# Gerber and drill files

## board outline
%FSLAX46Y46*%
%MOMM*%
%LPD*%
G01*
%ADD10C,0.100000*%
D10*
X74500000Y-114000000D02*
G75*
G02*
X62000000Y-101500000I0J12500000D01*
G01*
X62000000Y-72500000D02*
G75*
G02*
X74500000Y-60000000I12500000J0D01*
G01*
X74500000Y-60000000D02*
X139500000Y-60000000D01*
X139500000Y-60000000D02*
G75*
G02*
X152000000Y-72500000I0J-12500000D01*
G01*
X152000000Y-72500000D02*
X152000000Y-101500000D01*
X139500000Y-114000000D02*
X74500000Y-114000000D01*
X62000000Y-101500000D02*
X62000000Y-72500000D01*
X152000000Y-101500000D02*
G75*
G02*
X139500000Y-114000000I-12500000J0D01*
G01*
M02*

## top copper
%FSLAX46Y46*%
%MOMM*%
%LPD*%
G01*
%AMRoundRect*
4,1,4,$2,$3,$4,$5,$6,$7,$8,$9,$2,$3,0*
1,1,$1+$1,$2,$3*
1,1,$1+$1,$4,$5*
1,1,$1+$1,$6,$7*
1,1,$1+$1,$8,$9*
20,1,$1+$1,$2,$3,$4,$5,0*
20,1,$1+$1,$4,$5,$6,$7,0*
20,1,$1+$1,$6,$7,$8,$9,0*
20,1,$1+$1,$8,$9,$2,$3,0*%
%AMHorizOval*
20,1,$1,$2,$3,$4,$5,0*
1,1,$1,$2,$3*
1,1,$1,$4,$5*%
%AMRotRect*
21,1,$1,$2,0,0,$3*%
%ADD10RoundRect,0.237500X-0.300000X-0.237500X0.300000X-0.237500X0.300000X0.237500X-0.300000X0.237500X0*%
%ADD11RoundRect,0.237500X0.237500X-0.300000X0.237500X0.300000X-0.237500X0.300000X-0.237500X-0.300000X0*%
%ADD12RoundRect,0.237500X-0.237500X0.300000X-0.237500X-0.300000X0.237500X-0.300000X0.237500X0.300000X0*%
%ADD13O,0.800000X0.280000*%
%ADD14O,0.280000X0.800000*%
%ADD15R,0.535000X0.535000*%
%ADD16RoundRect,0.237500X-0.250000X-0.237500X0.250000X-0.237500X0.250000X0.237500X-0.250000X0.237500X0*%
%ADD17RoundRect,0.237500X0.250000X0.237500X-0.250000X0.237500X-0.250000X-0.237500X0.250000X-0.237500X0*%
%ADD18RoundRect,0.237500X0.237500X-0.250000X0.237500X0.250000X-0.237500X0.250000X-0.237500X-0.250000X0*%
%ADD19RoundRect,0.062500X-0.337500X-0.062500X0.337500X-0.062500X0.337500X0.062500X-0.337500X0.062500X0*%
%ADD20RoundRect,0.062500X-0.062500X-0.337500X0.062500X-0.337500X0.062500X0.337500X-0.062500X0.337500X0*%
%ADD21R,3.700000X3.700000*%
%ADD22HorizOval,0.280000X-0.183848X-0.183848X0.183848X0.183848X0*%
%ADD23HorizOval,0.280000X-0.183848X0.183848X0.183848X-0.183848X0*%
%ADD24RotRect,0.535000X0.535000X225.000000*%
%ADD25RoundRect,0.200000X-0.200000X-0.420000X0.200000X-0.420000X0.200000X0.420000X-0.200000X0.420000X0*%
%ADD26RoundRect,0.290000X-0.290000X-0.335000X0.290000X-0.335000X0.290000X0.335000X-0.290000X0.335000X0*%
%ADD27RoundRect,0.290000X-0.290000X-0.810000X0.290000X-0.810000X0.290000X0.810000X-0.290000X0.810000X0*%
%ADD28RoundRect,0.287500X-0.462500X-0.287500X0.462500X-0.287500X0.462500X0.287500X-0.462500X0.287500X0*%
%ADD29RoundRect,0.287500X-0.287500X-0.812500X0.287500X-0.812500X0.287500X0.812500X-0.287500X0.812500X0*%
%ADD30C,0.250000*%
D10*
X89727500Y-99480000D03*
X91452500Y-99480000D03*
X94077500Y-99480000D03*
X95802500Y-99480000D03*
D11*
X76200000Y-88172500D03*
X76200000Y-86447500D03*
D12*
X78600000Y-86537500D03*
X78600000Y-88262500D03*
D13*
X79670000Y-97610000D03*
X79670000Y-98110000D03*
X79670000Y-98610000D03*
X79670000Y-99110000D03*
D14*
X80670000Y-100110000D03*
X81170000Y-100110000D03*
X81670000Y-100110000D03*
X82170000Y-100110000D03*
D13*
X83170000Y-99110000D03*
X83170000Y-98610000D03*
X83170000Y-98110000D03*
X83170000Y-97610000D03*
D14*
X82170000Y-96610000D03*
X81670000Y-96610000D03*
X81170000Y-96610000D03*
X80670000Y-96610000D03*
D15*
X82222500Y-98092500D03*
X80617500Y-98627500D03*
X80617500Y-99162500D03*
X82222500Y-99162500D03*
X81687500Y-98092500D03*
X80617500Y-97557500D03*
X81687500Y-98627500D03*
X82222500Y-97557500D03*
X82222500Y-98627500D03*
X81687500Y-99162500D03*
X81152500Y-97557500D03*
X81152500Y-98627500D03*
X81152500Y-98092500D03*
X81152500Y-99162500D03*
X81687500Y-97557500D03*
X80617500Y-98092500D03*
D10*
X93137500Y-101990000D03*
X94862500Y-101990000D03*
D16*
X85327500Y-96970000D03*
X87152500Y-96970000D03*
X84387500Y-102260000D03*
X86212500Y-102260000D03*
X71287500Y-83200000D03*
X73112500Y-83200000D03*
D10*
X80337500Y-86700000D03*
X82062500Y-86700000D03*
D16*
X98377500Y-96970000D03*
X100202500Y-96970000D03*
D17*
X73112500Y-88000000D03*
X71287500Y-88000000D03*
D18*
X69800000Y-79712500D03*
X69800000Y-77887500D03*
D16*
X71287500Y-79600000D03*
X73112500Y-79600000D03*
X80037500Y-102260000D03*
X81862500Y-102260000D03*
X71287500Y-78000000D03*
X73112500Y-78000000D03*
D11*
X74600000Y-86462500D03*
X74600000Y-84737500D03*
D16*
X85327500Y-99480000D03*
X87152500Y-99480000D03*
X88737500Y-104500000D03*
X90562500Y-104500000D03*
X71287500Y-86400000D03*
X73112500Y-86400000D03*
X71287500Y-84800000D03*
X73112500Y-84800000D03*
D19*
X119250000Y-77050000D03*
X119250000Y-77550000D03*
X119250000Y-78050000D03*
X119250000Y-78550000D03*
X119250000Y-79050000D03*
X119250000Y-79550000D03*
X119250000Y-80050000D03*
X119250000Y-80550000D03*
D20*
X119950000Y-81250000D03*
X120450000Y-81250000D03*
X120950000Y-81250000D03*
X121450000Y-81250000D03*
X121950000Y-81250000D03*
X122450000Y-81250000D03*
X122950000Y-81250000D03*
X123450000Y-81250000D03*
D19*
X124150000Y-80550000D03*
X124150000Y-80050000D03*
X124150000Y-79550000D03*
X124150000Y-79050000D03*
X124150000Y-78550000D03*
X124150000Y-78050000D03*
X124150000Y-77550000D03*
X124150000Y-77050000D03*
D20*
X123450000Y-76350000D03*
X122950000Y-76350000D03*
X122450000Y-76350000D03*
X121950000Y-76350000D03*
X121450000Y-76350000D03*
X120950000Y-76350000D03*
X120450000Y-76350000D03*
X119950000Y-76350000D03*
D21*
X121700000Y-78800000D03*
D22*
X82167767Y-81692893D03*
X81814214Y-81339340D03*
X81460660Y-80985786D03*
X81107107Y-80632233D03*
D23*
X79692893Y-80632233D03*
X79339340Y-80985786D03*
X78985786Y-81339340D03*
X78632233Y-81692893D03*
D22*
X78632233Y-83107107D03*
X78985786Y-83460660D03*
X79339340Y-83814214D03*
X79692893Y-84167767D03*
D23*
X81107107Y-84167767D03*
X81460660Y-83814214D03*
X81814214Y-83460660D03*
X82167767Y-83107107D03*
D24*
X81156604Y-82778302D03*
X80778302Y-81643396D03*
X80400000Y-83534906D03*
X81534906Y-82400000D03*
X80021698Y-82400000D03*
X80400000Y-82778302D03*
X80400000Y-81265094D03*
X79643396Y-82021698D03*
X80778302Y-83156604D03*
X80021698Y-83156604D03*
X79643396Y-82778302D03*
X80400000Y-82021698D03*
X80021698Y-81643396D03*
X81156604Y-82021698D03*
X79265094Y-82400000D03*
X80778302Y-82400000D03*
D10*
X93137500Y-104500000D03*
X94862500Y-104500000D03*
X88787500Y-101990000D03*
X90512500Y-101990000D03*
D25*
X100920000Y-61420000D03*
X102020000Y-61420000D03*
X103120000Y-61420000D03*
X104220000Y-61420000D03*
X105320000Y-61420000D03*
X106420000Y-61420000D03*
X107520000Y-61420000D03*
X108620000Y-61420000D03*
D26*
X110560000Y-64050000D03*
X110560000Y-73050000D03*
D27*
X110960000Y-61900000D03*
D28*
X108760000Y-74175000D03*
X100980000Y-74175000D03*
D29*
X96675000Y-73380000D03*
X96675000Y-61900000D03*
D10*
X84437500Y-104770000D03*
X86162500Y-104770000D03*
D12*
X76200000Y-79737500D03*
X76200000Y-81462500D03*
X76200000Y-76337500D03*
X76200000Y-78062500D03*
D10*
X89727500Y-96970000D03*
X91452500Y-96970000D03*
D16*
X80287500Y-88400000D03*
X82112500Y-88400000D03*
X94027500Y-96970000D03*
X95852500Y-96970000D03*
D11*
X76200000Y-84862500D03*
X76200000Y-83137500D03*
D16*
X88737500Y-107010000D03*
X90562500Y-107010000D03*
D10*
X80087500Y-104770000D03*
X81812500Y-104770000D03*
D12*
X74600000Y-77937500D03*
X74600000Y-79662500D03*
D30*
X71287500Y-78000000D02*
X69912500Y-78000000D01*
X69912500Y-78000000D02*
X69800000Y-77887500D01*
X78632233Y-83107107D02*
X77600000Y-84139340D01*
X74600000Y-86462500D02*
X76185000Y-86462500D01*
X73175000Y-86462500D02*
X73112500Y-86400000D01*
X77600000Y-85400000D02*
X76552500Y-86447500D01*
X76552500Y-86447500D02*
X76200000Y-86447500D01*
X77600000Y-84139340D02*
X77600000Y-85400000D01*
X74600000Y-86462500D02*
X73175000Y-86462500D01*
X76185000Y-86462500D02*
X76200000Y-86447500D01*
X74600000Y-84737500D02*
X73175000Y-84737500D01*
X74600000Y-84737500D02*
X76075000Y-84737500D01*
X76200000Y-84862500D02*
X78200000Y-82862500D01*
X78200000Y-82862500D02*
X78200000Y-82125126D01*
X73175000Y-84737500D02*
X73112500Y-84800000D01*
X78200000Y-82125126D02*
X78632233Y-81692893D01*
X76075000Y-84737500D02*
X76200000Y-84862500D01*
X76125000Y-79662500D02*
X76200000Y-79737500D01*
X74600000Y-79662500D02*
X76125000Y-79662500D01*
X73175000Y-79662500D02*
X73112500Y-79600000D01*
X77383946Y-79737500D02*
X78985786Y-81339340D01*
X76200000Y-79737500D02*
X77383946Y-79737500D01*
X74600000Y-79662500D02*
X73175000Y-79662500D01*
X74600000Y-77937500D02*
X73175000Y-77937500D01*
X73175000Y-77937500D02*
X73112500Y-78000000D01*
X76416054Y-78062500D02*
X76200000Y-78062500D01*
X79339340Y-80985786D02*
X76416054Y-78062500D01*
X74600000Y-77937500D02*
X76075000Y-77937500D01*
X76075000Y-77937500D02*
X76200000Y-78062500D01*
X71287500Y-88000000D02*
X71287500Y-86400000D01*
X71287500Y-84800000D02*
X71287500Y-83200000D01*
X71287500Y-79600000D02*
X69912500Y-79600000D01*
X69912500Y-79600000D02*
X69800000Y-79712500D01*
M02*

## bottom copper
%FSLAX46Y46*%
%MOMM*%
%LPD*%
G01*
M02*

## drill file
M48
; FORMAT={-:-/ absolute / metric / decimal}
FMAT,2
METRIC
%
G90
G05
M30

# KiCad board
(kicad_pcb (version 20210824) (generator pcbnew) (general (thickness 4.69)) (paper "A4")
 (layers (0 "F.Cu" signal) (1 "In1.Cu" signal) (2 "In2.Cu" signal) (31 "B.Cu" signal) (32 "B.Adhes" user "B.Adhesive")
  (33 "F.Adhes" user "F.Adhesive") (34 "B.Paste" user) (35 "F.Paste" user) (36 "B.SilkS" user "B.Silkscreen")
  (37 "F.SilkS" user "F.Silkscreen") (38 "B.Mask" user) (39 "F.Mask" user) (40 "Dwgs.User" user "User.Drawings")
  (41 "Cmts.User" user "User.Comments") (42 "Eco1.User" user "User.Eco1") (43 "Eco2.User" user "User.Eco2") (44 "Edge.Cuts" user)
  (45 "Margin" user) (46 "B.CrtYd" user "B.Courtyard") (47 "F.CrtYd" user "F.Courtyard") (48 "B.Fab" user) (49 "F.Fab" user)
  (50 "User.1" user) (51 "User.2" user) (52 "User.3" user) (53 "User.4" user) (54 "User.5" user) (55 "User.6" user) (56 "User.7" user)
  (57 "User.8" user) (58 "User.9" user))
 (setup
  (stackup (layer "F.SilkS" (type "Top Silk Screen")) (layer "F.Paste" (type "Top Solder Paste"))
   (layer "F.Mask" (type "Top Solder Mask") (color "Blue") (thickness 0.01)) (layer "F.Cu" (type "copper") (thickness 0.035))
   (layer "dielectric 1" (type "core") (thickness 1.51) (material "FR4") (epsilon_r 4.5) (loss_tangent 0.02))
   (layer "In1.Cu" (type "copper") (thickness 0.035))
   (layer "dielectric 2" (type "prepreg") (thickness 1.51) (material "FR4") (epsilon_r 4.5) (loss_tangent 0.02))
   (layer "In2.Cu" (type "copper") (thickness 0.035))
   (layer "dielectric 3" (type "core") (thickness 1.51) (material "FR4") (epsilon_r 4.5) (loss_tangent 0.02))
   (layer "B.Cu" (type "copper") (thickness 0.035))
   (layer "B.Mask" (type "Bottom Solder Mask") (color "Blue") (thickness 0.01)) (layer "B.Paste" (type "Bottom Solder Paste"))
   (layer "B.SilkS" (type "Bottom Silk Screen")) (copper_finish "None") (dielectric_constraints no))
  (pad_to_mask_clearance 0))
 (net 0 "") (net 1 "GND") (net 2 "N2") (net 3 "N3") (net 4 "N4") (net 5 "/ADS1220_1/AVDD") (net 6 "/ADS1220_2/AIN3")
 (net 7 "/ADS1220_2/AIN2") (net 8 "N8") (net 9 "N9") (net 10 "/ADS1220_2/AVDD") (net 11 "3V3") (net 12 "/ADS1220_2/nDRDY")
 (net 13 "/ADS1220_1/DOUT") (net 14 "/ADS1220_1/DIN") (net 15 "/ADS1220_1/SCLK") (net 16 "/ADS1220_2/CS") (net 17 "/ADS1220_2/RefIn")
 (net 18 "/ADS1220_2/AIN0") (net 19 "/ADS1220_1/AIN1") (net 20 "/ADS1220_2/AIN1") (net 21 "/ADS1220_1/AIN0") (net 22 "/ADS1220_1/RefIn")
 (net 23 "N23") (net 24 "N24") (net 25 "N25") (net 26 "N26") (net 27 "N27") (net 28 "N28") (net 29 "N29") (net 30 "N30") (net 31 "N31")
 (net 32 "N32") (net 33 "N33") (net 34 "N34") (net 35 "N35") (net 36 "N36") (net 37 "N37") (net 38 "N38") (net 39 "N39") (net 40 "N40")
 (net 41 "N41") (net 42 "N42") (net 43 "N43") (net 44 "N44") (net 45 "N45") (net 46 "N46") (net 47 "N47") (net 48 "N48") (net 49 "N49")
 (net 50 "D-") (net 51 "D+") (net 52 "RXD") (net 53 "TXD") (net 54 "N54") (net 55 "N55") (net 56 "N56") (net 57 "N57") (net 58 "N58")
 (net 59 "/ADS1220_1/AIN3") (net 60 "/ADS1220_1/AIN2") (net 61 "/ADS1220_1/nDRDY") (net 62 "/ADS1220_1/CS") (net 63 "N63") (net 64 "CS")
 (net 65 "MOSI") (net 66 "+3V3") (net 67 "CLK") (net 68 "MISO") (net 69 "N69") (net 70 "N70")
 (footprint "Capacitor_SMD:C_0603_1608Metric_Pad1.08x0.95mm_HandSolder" (layer "F.Cu") (at 90.59 99.48)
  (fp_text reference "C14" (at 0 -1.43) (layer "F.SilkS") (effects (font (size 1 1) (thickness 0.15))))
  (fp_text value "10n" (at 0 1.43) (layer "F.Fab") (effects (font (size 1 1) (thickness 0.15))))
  (pad "1" smd roundrect locked (at -0.8625 0) (size 1.075 0.95) (layers "F.Cu" "F.Paste" "F.Mask") (roundrect_rratio 0.25) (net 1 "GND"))
  (pad "2" smd roundrect locked (at 0.8625 0) (size 1.075 0.95) (layers "F.Cu" "F.Paste" "F.Mask") (roundrect_rratio 0.25) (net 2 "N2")))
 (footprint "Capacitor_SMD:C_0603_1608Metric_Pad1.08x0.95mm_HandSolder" (layer "F.Cu") (at 94.94 99.48)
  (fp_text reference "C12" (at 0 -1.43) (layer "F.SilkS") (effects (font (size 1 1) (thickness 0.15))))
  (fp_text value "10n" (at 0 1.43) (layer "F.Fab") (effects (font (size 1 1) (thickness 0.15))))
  (pad "1" smd roundrect locked (at -0.8625 0) (size 1.075 0.95) (layers "F.Cu" "F.Paste" "F.Mask") (roundrect_rratio 0.25) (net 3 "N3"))
  (pad "2" smd roundrect locked (at 0.8625 0) (size 1.075 0.95) (layers "F.Cu" "F.Paste" "F.Mask") (roundrect_rratio 0.25) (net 1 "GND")))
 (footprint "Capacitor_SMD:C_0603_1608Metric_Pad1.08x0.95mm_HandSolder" (layer "F.Cu") (at 76.2 87.31 90)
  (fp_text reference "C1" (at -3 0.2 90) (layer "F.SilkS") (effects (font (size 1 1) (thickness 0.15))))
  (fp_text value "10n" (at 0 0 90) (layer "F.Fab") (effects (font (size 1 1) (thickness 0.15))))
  (pad "1" smd roundrect locked (at -0.8625 0 90) (size 1.075 0.95) (layers "F.Cu" "F.Paste" "F.Mask") (roundrect_rratio 0.25) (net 1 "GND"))
  (pad "2" smd roundrect locked (at 0.8625 0 90) (size 1.075 0.95) (layers "F.Cu" "F.Paste" "F.Mask") (roundrect_rratio 0.25) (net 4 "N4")))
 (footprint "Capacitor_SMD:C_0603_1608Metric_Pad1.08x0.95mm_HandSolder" (layer "F.Cu") (at 78.6 87.4 -90)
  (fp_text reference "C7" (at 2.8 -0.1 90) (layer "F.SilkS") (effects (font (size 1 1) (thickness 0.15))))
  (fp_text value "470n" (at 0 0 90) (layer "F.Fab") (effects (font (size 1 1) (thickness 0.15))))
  (pad "1" smd roundrect locked (at -0.8625 0 270) (size 1.075 0.95) (layers "F.Cu" "F.Paste" "F.Mask") (roundrect_rratio 0.25)
   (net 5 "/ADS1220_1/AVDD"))
  (pad "2" smd roundrect locked (at 0.8625 0 270) (size 1.075 0.95) (layers "F.Cu" "F.Paste" "F.Mask") (roundrect_rratio 0.25) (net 1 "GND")))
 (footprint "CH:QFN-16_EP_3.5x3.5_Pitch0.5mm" (layer "F.Cu") (at 81.42 98.36)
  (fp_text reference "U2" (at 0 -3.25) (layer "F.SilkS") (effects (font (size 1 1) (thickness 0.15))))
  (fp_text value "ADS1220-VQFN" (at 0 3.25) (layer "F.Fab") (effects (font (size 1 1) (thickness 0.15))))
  (pad "1" smd oval (at -1.75 -0.75 90) (size 0.28 0.8) (layers "F.Cu" "F.Paste" "F.Mask") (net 1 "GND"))
  (pad "2" smd oval (at -1.75 -0.25 90) (size 0.28 0.8) (layers "F.Cu" "F.Paste" "F.Mask") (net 1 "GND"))
  (pad "3" smd oval (at -1.75 0.25 90) (size 0.28 0.8) (layers "F.Cu" "F.Paste" "F.Mask") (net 1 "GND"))
  (pad "4" smd oval (at -1.75 0.75 90) (size 0.28 0.8) (layers "F.Cu" "F.Paste" "F.Mask") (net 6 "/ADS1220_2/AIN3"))
  (pad "5" smd oval (at -0.75 1.75) (size 0.28 0.8) (layers "F.Cu" "F.Paste" "F.Mask") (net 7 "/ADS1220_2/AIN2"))
  (pad "6" smd oval (at -0.25 1.75) (size 0.28 0.8) (layers "F.Cu" "F.Paste" "F.Mask") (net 2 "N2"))
  (pad "7" smd oval (at 0.25 1.75) (size 0.28 0.8) (layers "F.Cu" "F.Paste" "F.Mask") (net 3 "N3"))
  (pad "8" smd oval (at 0.75 1.75) (size 0.28 0.8) (layers "F.Cu" "F.Paste" "F.Mask") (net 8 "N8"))
  (pad "9" smd oval (at 1.75 0.75 90) (size 0.28 0.8) (layers "F.Cu" "F.Paste" "F.Mask") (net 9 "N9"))
  (pad "10" smd oval (at 1.75 0.25 90) (size 0.28 0.8) (layers "F.Cu" "F.Paste" "F.Mask") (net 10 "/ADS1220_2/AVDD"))
  (pad "11" smd oval (at 1.75 -0.25 90) (size 0.28 0.8) (layers "F.Cu" "F.Paste" "F.Mask") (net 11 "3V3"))
  (pad "12" smd oval (at 1.75 -0.75 90) (size 0.28 0.8) (layers "F.Cu" "F.Paste" "F.Mask") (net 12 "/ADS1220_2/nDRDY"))
  (pad "13" smd oval (at 0.75 -1.75) (size 0.28 0.8) (layers "F.Cu" "F.Paste" "F.Mask") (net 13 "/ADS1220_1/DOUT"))
  (pad "14" smd oval (at 0.25 -1.75) (size 0.28 0.8) (layers "F.Cu" "F.Paste" "F.Mask") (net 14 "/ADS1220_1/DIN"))
  (pad "15" smd oval (at -0.25 -1.75) (size 0.28 0.8) (layers "F.Cu" "F.Paste" "F.Mask") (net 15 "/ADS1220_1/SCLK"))
  (pad "16" smd oval (at -0.75 -1.75) (size 0.28 0.8) (layers "F.Cu" "F.Paste" "F.Mask") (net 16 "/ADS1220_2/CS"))
  (pad "17" smd rect (at 0.8025 -0.2675) (size 0.535 0.535) (layers "F.Cu" "F.Paste" "F.Mask") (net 1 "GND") (solder_paste_margin -0.75))
  (pad "17" smd rect (at -0.8025 0.2675) (size 0.535 0.535) (layers "F.Cu" "F.Paste" "F.Mask") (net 1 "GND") (solder_paste_margin -0.75))
  (pad "17" smd rect (at -0.8025 0.8025) (size 0.535 0.535) (layers "F.Cu" "F.Paste" "F.Mask") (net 1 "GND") (solder_paste_margin -0.75))
  (pad "17" smd rect (at 0.8025 0.8025) (size 0.535 0.535) (layers "F.Cu" "F.Paste" "F.Mask") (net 1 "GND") (solder_paste_margin -0.75))
  (pad "17" smd rect (at 0.2675 -0.2675) (size 0.535 0.535) (layers "F.Cu" "F.Paste" "F.Mask") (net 1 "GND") (solder_paste_margin -0.75))
  (pad "17" smd rect (at -0.8025 -0.8025) (size 0.535 0.535) (layers "F.Cu" "F.Paste" "F.Mask") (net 1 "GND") (solder_paste_margin -0.75))
  (pad "17" smd rect (at 0.2675 0.2675) (size 0.535 0.535) (layers "F.Cu" "F.Paste" "F.Mask") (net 1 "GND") (solder_paste_margin -0.75))
  (pad "17" smd rect (at 0.8025 -0.8025) (size 0.535 0.535) (layers "F.Cu" "F.Paste" "F.Mask") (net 1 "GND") (solder_paste_margin -0.75))
  (pad "17" smd rect (at 0.8025 0.2675) (size 0.535 0.535) (layers "F.Cu" "F.Paste" "F.Mask") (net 1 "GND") (solder_paste_margin -0.75))
  (pad "17" smd rect (at 0.2675 0.8025) (size 0.535 0.535) (layers "F.Cu" "F.Paste" "F.Mask") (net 1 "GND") (solder_paste_margin -0.75))
  (pad "17" smd rect (at -0.2675 -0.8025) (size 0.535 0.535) (layers "F.Cu" "F.Paste" "F.Mask") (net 1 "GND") (solder_paste_margin -0.75))
  (pad "17" smd rect (at -0.2675 0.2675) (size 0.535 0.535) (layers "F.Cu" "F.Paste" "F.Mask") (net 1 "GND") (solder_paste_margin -0.75))
  (pad "17" smd rect (at -0.2675 -0.2675) (size 0.535 0.535) (layers "F.Cu" "F.Paste" "F.Mask") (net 1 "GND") (solder_paste_margin -0.75))
  (pad "17" smd rect (at -0.2675 0.8025) (size 0.535 0.535) (layers "F.Cu" "F.Paste" "F.Mask") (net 1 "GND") (solder_paste_margin -0.75))
  (pad "17" smd rect (at 0.2675 -0.8025) (size 0.535 0.535) (layers "F.Cu" "F.Paste" "F.Mask") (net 1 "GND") (solder_paste_margin -0.75))
  (pad "17" smd rect (at -0.8025 -0.2675) (size 0.535 0.535) (layers "F.Cu" "F.Paste" "F.Mask") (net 1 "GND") (solder_paste_margin -0.75)))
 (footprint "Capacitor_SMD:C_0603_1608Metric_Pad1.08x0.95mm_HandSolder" (layer "F.Cu") (at 94 101.99)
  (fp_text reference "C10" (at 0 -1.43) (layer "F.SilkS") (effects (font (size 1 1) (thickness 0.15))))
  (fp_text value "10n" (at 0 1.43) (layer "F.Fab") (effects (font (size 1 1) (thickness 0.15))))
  (pad "1" smd roundrect locked (at -0.8625 0) (size 1.075 0.95) (layers "F.Cu" "F.Paste" "F.Mask") (roundrect_rratio 0.25) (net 8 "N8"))
  (pad "2" smd roundrect locked (at 0.8625 0) (size 1.075 0.95) (layers "F.Cu" "F.Paste" "F.Mask") (roundrect_rratio 0.25) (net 1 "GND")))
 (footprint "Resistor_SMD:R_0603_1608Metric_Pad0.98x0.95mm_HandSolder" (layer "F.Cu") (at 86.24 96.97)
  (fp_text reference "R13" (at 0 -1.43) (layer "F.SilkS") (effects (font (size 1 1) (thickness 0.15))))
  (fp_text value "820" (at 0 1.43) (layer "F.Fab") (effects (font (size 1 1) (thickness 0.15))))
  (pad "1" smd roundrect locked (at -0.9125 0) (size 0.975 0.95) (layers "F.Cu" "F.Paste" "F.Mask") (roundrect_rratio 0.25)
   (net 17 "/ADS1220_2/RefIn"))
  (pad "2" smd roundrect locked (at 0.9125 0) (size 0.975 0.95) (layers "F.Cu" "F.Paste" "F.Mask") (roundrect_rratio 0.25) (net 3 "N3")))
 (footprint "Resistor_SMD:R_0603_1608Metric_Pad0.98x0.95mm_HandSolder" (layer "F.Cu") (at 85.3 102.26)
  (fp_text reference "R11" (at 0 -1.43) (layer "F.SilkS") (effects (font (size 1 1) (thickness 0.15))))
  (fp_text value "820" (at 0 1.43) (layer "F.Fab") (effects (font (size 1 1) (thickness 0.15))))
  (pad "1" smd roundrect locked (at -0.9125 0) (size 0.975 0.95) (layers "F.Cu" "F.Paste" "F.Mask") (roundrect_rratio 0.25)
   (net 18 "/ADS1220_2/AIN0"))
  (pad "2" smd roundrect locked (at 0.9125 0) (size 0.975 0.95) (layers "F.Cu" "F.Paste" "F.Mask") (roundrect_rratio 0.25) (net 9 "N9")))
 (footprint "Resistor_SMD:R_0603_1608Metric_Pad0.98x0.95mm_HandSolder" (layer "F.Cu") (at 72.2 83.2)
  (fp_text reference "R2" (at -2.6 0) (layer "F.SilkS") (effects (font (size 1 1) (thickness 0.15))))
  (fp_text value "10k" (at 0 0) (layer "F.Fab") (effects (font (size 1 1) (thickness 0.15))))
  (pad "1" smd roundrect locked (at -0.9125 0) (size 0.975 0.95) (layers "F.Cu" "F.Paste" "F.Mask") (roundrect_rratio 0.25)
   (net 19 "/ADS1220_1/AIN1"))
  (pad "2" smd roundrect locked (at 0.9125 0) (size 0.975 0.95) (layers "F.Cu" "F.Paste" "F.Mask") (roundrect_rratio 0.25) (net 1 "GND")))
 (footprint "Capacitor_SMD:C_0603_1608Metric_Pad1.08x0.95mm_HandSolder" (layer "F.Cu") (at 81.2 86.7)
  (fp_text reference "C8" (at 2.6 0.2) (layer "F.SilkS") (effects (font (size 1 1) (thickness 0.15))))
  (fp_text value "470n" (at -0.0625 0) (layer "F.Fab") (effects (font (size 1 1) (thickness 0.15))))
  (pad "1" smd roundrect locked (at -0.8625 0) (size 1.075 0.95) (layers "F.Cu" "F.Paste" "F.Mask") (roundrect_rratio 0.25) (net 11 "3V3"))
  (pad "2" smd roundrect locked (at 0.8625 0) (size 1.075 0.95) (layers "F.Cu" "F.Paste" "F.Mask") (roundrect_rratio 0.25) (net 1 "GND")))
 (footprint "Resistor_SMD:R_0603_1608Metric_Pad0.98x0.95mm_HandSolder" (layer "F.Cu") (at 99.29 96.97)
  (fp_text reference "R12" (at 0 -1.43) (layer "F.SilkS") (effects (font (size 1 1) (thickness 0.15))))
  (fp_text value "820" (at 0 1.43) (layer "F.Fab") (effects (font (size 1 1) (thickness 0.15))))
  (pad "1" smd roundrect locked (at -0.9125 0) (size 0.975 0.95) (layers "F.Cu" "F.Paste" "F.Mask") (roundrect_rratio 0.25)
   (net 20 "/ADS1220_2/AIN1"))
  (pad "2" smd roundrect locked (at 0.9125 0) (size 0.975 0.95) (layers "F.Cu" "F.Paste" "F.Mask") (roundrect_rratio 0.25) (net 8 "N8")))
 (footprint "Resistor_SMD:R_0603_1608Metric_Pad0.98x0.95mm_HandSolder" (layer "F.Cu") (at 72.2 88 180)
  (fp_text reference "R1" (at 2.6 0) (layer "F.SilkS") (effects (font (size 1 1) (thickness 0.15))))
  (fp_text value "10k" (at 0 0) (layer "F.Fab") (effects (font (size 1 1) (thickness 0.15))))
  (pad "1" smd roundrect locked (at -0.9125 0 180) (size 0.975 0.95) (layers "F.Cu" "F.Paste" "F.Mask") (roundrect_rratio 0.25)
   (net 5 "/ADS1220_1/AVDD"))
  (pad "2" smd roundrect locked (at 0.9125 0 180) (size 0.975 0.95) (layers "F.Cu" "F.Paste" "F.Mask") (roundrect_rratio 0.25)
   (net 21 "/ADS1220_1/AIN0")))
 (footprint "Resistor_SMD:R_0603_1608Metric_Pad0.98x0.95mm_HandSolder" (layer "F.Cu") (at 69.8 78.8 90)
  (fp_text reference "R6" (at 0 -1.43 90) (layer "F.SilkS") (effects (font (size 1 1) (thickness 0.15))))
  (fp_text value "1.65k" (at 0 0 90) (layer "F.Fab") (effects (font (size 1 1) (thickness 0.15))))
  (pad "1" smd roundrect locked (at -0.9125 0 90) (size 0.975 0.95) (layers "F.Cu" "F.Paste" "F.Mask") (roundrect_rratio 0.25)
   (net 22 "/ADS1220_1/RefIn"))
  (pad "2" smd roundrect locked (at 0.9125 0 90) (size 0.975 0.95) (layers "F.Cu" "F.Paste" "F.Mask") (roundrect_rratio 0.25) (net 1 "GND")))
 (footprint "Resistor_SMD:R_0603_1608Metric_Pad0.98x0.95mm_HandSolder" (layer "F.Cu") (at 72.2 79.6)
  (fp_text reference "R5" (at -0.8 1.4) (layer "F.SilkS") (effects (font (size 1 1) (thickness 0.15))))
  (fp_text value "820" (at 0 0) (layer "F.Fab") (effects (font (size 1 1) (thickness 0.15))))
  (pad "1" smd roundrect locked (at -0.9125 0) (size 0.975 0.95) (layers "F.Cu" "F.Paste" "F.Mask") (roundrect_rratio 0.25)
   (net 22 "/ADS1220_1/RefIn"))
  (pad "2" smd roundrect locked (at 0.9125 0) (size 0.975 0.95) (layers "F.Cu" "F.Paste" "F.Mask") (roundrect_rratio 0.25) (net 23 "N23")))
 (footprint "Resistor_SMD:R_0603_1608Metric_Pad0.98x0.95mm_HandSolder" (layer "F.Cu") (at 80.95 102.26)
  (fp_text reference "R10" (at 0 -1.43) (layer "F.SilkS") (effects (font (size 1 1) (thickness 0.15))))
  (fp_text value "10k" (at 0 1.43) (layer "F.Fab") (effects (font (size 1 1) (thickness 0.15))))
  (pad "1" smd roundrect locked (at -0.9125 0) (size 0.975 0.95) (layers "F.Cu" "F.Paste" "F.Mask") (roundrect_rratio 0.25)
   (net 20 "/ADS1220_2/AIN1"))
  (pad "2" smd roundrect locked (at 0.9125 0) (size 0.975 0.95) (layers "F.Cu" "F.Paste" "F.Mask") (roundrect_rratio 0.25) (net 1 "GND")))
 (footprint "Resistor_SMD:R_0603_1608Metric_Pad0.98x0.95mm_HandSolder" (layer "F.Cu") (at 72.2 78)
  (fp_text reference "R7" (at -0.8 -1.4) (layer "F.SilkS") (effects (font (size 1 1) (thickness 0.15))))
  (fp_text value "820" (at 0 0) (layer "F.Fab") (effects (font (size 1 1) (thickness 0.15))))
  (pad "1" smd roundrect locked (at -0.9125 0) (size 0.975 0.95) (layers "F.Cu" "F.Paste" "F.Mask") (roundrect_rratio 0.25) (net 1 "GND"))
  (pad "2" smd roundrect locked (at 0.9125 0) (size 0.975 0.95) (layers "F.Cu" "F.Paste" "F.Mask") (roundrect_rratio 0.25) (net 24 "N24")))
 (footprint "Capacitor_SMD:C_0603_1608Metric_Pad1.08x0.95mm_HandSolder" (layer "F.Cu") (at 74.6 85.6 90)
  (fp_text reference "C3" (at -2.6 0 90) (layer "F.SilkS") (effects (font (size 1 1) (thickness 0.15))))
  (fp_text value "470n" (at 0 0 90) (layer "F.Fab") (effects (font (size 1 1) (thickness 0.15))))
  (pad "1" smd roundrect locked (at -0.8625 0 90) (size 1.075 0.95) (layers "F.Cu" "F.Paste" "F.Mask") (roundrect_rratio 0.25) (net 4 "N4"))
  (pad "2" smd roundrect locked (at 0.8625 0 90) (size 1.075 0.95) (layers "F.Cu" "F.Paste" "F.Mask") (roundrect_rratio 0.25) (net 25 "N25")))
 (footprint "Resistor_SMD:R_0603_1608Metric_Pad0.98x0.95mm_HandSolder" (layer "F.Cu") (at 86.24 99.48)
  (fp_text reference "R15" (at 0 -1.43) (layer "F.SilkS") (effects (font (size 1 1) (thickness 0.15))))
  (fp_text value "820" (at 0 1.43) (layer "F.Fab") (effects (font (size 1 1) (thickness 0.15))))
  (pad "1" smd roundrect locked (at -0.9125 0) (size 0.975 0.95) (layers "F.Cu" "F.Paste" "F.Mask") (roundrect_rratio 0.25) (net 1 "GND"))
  (pad "2" smd roundrect locked (at 0.9125 0) (size 0.975 0.95) (layers "F.Cu" "F.Paste" "F.Mask") (roundrect_rratio 0.25) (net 2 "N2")))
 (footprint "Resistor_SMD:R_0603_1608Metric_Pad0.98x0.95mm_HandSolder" (layer "F.Cu") (at 89.65 104.5)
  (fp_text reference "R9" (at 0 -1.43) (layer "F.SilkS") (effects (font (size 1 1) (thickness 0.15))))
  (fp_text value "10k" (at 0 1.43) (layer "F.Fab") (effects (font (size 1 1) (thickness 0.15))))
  (pad "1" smd roundrect locked (at -0.9125 0) (size 0.975 0.95) (layers "F.Cu" "F.Paste" "F.Mask") (roundrect_rratio 0.25)
   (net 10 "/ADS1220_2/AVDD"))
  (pad "2" smd roundrect locked (at 0.9125 0) (size 0.975 0.95) (layers "F.Cu" "F.Paste" "F.Mask") (roundrect_rratio 0.25)
   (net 18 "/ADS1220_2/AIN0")))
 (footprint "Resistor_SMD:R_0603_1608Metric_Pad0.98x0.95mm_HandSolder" (layer "F.Cu") (at 72.2 86.4)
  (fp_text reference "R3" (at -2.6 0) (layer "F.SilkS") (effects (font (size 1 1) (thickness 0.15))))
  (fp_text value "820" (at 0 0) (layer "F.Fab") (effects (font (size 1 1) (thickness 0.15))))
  (pad "1" smd roundrect locked (at -0.9125 0) (size 0.975 0.95) (layers "F.Cu" "F.Paste" "F.Mask") (roundrect_rratio 0.25)
   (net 21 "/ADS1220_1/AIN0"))
  (pad "2" smd roundrect locked (at 0.9125 0) (size 0.975 0.95) (layers "F.Cu" "F.Paste" "F.Mask") (roundrect_rratio 0.25) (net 4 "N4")))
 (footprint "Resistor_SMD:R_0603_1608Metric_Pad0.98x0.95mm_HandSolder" (layer "F.Cu") (at 72.2 84.8)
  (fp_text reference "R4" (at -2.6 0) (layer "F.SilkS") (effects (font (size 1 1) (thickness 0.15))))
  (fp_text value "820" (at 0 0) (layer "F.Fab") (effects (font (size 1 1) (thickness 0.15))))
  (pad "1" smd roundrect locked (at -0.9125 0) (size 0.975 0.95) (layers "F.Cu" "F.Paste" "F.Mask") (roundrect_rratio 0.25)
   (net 19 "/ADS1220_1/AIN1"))
  (pad "2" smd roundrect locked (at 0.9125 0) (size 0.975 0.95) (layers "F.Cu" "F.Paste" "F.Mask") (roundrect_rratio 0.25) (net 25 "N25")))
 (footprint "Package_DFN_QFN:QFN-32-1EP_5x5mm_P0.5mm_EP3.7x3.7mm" (layer "F.Cu") (at 121.7 78.8)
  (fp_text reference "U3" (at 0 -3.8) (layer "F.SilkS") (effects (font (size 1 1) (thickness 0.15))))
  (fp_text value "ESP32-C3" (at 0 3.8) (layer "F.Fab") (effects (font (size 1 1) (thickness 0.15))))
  (pad "" smd roundrect locked (at 0.925 -0.925) (size 1.49 1.49) (layers "F.Paste") (roundrect_rratio 0.167785))
  (pad "" smd roundrect locked (at -0.925 0.925) (size 1.49 1.49) (layers "F.Paste") (roundrect_rratio 0.167785))
  (pad "" smd roundrect locked (at -0.925 -0.925) (size 1.49 1.49) (layers "F.Paste") (roundrect_rratio 0.167785))
  (pad "" smd roundrect locked (at 0.925 0.925) (size 1.49 1.49) (layers "F.Paste") (roundrect_rratio 0.167785))
  (pad "1" smd roundrect locked (at -2.45 -1.75) (size 0.8 0.25) (layers "F.Cu" "F.Paste" "F.Mask") (roundrect_rratio 0.25) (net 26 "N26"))
  (pad "2" smd roundrect locked (at -2.45 -1.25) (size 0.8 0.25) (layers "F.Cu" "F.Paste" "F.Mask") (roundrect_rratio 0.25) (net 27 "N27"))
  (pad "3" smd roundrect locked (at -2.45 -0.75) (size 0.8 0.25) (layers "F.Cu" "F.Paste" "F.Mask") (roundrect_rratio 0.25) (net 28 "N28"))
  (pad "4" smd roundrect locked (at -2.45 -0.25) (size 0.8 0.25) (layers "F.Cu" "F.Paste" "F.Mask") (roundrect_rratio 0.25) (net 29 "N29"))
  (pad "5" smd roundrect locked (at -2.45 0.25) (size 0.8 0.25) (layers "F.Cu" "F.Paste" "F.Mask") (roundrect_rratio 0.25) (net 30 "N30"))
  (pad "6" smd roundrect locked (at -2.45 0.75) (size 0.8 0.25) (layers "F.Cu" "F.Paste" "F.Mask") (roundrect_rratio 0.25) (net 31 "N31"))
  (pad "7" smd roundrect locked (at -2.45 1.25) (size 0.8 0.25) (layers "F.Cu" "F.Paste" "F.Mask") (roundrect_rratio 0.25) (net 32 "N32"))
  (pad "8" smd roundrect locked (at -2.45 1.75) (size 0.8 0.25) (layers "F.Cu" "F.Paste" "F.Mask") (roundrect_rratio 0.25) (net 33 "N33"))
  (pad "9" smd roundrect locked (at -1.75 2.45) (size 0.25 0.8) (layers "F.Cu" "F.Paste" "F.Mask") (roundrect_rratio 0.25) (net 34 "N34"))
  (pad "10" smd roundrect locked (at -1.25 2.45) (size 0.25 0.8) (layers "F.Cu" "F.Paste" "F.Mask") (roundrect_rratio 0.25) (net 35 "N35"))
  (pad "11" smd roundrect locked (at -0.75 2.45) (size 0.25 0.8) (layers "F.Cu" "F.Paste" "F.Mask") (roundrect_rratio 0.25) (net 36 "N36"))
  (pad "12" smd roundrect locked (at -0.25 2.45) (size 0.25 0.8) (layers "F.Cu" "F.Paste" "F.Mask") (roundrect_rratio 0.25) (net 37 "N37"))
  (pad "13" smd roundrect locked (at 0.25 2.45) (size 0.25 0.8) (layers "F.Cu" "F.Paste" "F.Mask") (roundrect_rratio 0.25) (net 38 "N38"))
  (pad "14" smd roundrect locked (at 0.75 2.45) (size 0.25 0.8) (layers "F.Cu" "F.Paste" "F.Mask") (roundrect_rratio 0.25) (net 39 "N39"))
  (pad "15" smd roundrect locked (at 1.25 2.45) (size 0.25 0.8) (layers "F.Cu" "F.Paste" "F.Mask") (roundrect_rratio 0.25) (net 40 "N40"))
  (pad "16" smd roundrect locked (at 1.75 2.45) (size 0.25 0.8) (layers "F.Cu" "F.Paste" "F.Mask") (roundrect_rratio 0.25) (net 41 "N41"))
  (pad "17" smd roundrect locked (at 2.45 1.75) (size 0.8 0.25) (layers "F.Cu" "F.Paste" "F.Mask") (roundrect_rratio 0.25) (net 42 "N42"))
  (pad "18" smd roundrect locked (at 2.45 1.25) (size 0.8 0.25) (layers "F.Cu" "F.Paste" "F.Mask") (roundrect_rratio 0.25) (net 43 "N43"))
  (pad "19" smd roundrect locked (at 2.45 0.75) (size 0.8 0.25) (layers "F.Cu" "F.Paste" "F.Mask") (roundrect_rratio 0.25) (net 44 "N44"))
  (pad "20" smd roundrect locked (at 2.45 0.25) (size 0.8 0.25) (layers "F.Cu" "F.Paste" "F.Mask") (roundrect_rratio 0.25) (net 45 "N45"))
  (pad "21" smd roundrect locked (at 2.45 -0.25) (size 0.8 0.25) (layers "F.Cu" "F.Paste" "F.Mask") (roundrect_rratio 0.25) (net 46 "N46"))
  (pad "22" smd roundrect locked (at 2.45 -0.75) (size 0.8 0.25) (layers "F.Cu" "F.Paste" "F.Mask") (roundrect_rratio 0.25) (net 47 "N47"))
  (pad "23" smd roundrect locked (at 2.45 -1.25) (size 0.8 0.25) (layers "F.Cu" "F.Paste" "F.Mask") (roundrect_rratio 0.25) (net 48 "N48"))
  (pad "24" smd roundrect locked (at 2.45 -1.75) (size 0.8 0.25) (layers "F.Cu" "F.Paste" "F.Mask") (roundrect_rratio 0.25) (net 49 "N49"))
  (pad "25" smd roundrect locked (at 1.75 -2.45) (size 0.25 0.8) (layers "F.Cu" "F.Paste" "F.Mask") (roundrect_rratio 0.25) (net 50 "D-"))
  (pad "26" smd roundrect locked (at 1.25 -2.45) (size 0.25 0.8) (layers "F.Cu" "F.Paste" "F.Mask") (roundrect_rratio 0.25) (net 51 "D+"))
  (pad "27" smd roundrect locked (at 0.75 -2.45) (size 0.25 0.8) (layers "F.Cu" "F.Paste" "F.Mask") (roundrect_rratio 0.25) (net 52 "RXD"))
  (pad "28" smd roundrect locked (at 0.25 -2.45) (size 0.25 0.8) (layers "F.Cu" "F.Paste" "F.Mask") (roundrect_rratio 0.25) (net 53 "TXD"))
  (pad "29" smd roundrect locked (at -0.25 -2.45) (size 0.25 0.8) (layers "F.Cu" "F.Paste" "F.Mask") (roundrect_rratio 0.25) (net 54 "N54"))
  (pad "30" smd roundrect locked (at -0.75 -2.45) (size 0.25 0.8) (layers "F.Cu" "F.Paste" "F.Mask") (roundrect_rratio 0.25) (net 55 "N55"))
  (pad "31" smd roundrect locked (at -1.25 -2.45) (size 0.25 0.8) (layers "F.Cu" "F.Paste" "F.Mask") (roundrect_rratio 0.25) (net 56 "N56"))
  (pad "32" smd roundrect locked (at -1.75 -2.45) (size 0.25 0.8) (layers "F.Cu" "F.Paste" "F.Mask") (roundrect_rratio 0.25) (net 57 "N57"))
  (pad "33" smd rect locked (at 0 0) (size 3.7 3.7) (layers "F.Cu" "F.Mask") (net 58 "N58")))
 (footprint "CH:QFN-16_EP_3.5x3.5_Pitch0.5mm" (layer "F.Cu") (at 80.4 82.4 -135)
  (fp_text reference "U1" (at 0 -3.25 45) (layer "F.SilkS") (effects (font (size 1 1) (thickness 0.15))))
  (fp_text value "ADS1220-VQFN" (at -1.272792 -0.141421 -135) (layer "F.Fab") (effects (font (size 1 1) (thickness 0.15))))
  (pad "1" smd oval (at -1.75 -0.75 315) (size 0.28 0.8) (layers "F.Cu" "F.Paste" "F.Mask") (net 1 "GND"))
  (pad "2" smd oval (at -1.75 -0.25 315) (size 0.28 0.8) (layers "F.Cu" "F.Paste" "F.Mask") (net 1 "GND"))
  (pad "3" smd oval (at -1.75 0.25 315) (size 0.28 0.8) (layers "F.Cu" "F.Paste" "F.Mask") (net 1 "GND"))
  (pad "4" smd oval (at -1.75 0.75 315) (size 0.28 0.8) (layers "F.Cu" "F.Paste" "F.Mask") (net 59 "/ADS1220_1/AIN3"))
  (pad "5" smd oval (at -0.75 1.75 225) (size 0.28 0.8) (layers "F.Cu" "F.Paste" "F.Mask") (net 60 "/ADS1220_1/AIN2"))
  (pad "6" smd oval (at -0.25 1.75 225) (size 0.28 0.8) (layers "F.Cu" "F.Paste" "F.Mask") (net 24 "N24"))
  (pad "7" smd oval (at 0.25 1.75 225) (size 0.28 0.8) (layers "F.Cu" "F.Paste" "F.Mask") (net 23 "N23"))
  (pad "8" smd oval (at 0.75 1.75 225) (size 0.28 0.8) (layers "F.Cu" "F.Paste" "F.Mask") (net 25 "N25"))
  (pad "9" smd oval (at 1.75 0.75 315) (size 0.28 0.8) (layers "F.Cu" "F.Paste" "F.Mask") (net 4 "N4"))
  (pad "10" smd oval (at 1.75 0.25 315) (size 0.28 0.8) (layers "F.Cu" "F.Paste" "F.Mask") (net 5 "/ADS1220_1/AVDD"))
  (pad "11" smd oval (at 1.75 -0.25 315) (size 0.28 0.8) (layers "F.Cu" "F.Paste" "F.Mask") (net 11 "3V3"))
  (pad "12" smd oval (at 1.75 -0.75 315) (size 0.28 0.8) (layers "F.Cu" "F.Paste" "F.Mask") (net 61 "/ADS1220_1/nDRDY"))
  (pad "13" smd oval (at 0.75 -1.75 225) (size 0.28 0.8) (layers "F.Cu" "F.Paste" "F.Mask") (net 13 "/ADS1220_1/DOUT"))
  (pad "14" smd oval (at 0.25 -1.75 225) (size 0.28 0.8) (layers "F.Cu" "F.Paste" "F.Mask") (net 14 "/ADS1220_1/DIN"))
  (pad "15" smd oval (at -0.25 -1.75 225) (size 0.28 0.8) (layers "F.Cu" "F.Paste" "F.Mask") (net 15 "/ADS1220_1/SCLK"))
  (pad "16" smd oval (at -0.75 -1.75 225) (size 0.28 0.8) (layers "F.Cu" "F.Paste" "F.Mask") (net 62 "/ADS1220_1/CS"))
  (pad "17" smd rect (at -0.2675 -0.8025 225) (size 0.535 0.535) (layers "F.Cu" "F.Paste" "F.Mask") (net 1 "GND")
   (solder_paste_margin -0.75))
  (pad "17" smd rect (at -0.8025 0.2675 225) (size 0.535 0.535) (layers "F.Cu" "F.Paste" "F.Mask") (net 1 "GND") (solder_paste_margin -0.75))
  (pad "17" smd rect (at 0.8025 -0.8025 225) (size 0.535 0.535) (layers "F.Cu" "F.Paste" "F.Mask") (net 1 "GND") (solder_paste_margin -0.75))
  (pad "17" smd rect (at -0.8025 -0.8025 225) (size 0.535 0.535) (layers "F.Cu" "F.Paste" "F.Mask") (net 1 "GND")
   (solder_paste_margin -0.75))
  (pad "17" smd rect (at 0.2675 0.2675 225) (size 0.535 0.535) (layers "F.Cu" "F.Paste" "F.Mask") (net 1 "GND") (solder_paste_margin -0.75))
  (pad "17" smd rect (at 0.2675 -0.2675 225) (size 0.535 0.535) (layers "F.Cu" "F.Paste" "F.Mask") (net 1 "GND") (solder_paste_margin -0.75))
  (pad "17" smd rect (at -0.8025 0.8025 225) (size 0.535 0.535) (layers "F.Cu" "F.Paste" "F.Mask") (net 1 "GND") (solder_paste_margin -0.75))
  (pad "17" smd rect (at 0.2675 0.8025 225) (size 0.535 0.535) (layers "F.Cu" "F.Paste" "F.Mask") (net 1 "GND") (solder_paste_margin -0.75))
  (pad "17" smd rect (at 0.2675 -0.8025 225) (size 0.535 0.535) (layers "F.Cu" "F.Paste" "F.Mask") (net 1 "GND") (solder_paste_margin -0.75))
  (pad "17" smd rect (at 0.8025 -0.2675 225) (size 0.535 0.535) (layers "F.Cu" "F.Paste" "F.Mask") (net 1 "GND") (solder_paste_margin -0.75))
  (pad "17" smd rect (at 0.8025 0.2675 225) (size 0.535 0.535) (layers "F.Cu" "F.Paste" "F.Mask") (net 1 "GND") (solder_paste_margin -0.75))
  (pad "17" smd rect (at -0.2675 0.2675 225) (size 0.535 0.535) (layers "F.Cu" "F.Paste" "F.Mask") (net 1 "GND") (solder_paste_margin -0.75))
  (pad "17" smd rect (at -0.2675 0.8025 225) (size 0.535 0.535) (layers "F.Cu" "F.Paste" "F.Mask") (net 1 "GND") (solder_paste_margin -0.75))
  (pad "17" smd rect (at -0.8025 -0.2675 225) (size 0.535 0.535) (layers "F.Cu" "F.Paste" "F.Mask") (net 1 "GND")
   (solder_paste_margin -0.75))
  (pad "17" smd rect (at 0.8025 0.8025 225) (size 0.535 0.535) (layers "F.Cu" "F.Paste" "F.Mask") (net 1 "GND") (solder_paste_margin -0.75))
  (pad "17" smd rect (at -0.2675 -0.2675 225) (size 0.535 0.535) (layers "F.Cu" "F.Paste" "F.Mask") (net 1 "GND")
   (solder_paste_margin -0.75)))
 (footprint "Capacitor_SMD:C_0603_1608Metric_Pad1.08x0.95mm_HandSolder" (layer "F.Cu") (at 94 104.5)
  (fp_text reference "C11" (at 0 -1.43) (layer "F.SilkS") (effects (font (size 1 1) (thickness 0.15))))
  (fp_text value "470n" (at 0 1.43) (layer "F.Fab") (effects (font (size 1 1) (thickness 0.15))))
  (pad "1" smd roundrect locked (at -0.8625 0) (size 1.075 0.95) (layers "F.Cu" "F.Paste" "F.Mask") (roundrect_rratio 0.25) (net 9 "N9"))
  (pad "2" smd roundrect locked (at 0.8625 0) (size 1.075 0.95) (layers "F.Cu" "F.Paste" "F.Mask") (roundrect_rratio 0.25) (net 8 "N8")))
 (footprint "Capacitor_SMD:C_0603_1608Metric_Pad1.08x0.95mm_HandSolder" (layer "F.Cu") (at 89.65 101.99)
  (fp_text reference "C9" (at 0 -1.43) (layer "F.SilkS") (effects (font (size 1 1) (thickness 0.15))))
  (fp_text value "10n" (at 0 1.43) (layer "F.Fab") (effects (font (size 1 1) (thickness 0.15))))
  (pad "1" smd roundrect locked (at -0.8625 0) (size 1.075 0.95) (layers "F.Cu" "F.Paste" "F.Mask") (roundrect_rratio 0.25) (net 1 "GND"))
  (pad "2" smd roundrect locked (at 0.8625 0) (size 1.075 0.95) (layers "F.Cu" "F.Paste" "F.Mask") (roundrect_rratio 0.25) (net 9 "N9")))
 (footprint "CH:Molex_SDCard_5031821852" (layer "F.Cu") (at 96.1 60.8)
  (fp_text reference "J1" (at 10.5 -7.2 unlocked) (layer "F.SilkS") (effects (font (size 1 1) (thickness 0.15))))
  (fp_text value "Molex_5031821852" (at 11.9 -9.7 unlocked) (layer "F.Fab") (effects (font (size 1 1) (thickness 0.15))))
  (pad "1" smd roundrect (at 4.82 0.62) (size 0.8 1.24) (layers "F.Cu" "F.Paste" "F.Mask") (roundrect_rratio 0.25) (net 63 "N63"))
  (pad "2" smd roundrect (at 5.92 0.62) (size 0.8 1.24) (layers "F.Cu" "F.Paste" "F.Mask") (roundrect_rratio 0.25) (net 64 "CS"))
  (pad "3" smd roundrect (at 7.02 0.62) (size 0.8 1.24) (layers "F.Cu" "F.Paste" "F.Mask") (roundrect_rratio 0.25) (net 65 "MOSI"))
  (pad "4" smd roundrect (at 8.12 0.62) (size 0.8 1.24) (layers "F.Cu" "F.Paste" "F.Mask") (roundrect_rratio 0.25) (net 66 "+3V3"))
  (pad "5" smd roundrect (at 9.22 0.62) (size 0.8 1.24) (layers "F.Cu" "F.Paste" "F.Mask") (roundrect_rratio 0.25) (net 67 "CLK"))
  (pad "6" smd roundrect (at 10.32 0.62) (size 0.8 1.24) (layers "F.Cu" "F.Paste" "F.Mask") (roundrect_rratio 0.25) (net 1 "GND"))
  (pad "7" smd roundrect (at 11.42 0.62) (size 0.8 1.24) (layers "F.Cu" "F.Paste" "F.Mask") (roundrect_rratio 0.25) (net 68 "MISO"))
  (pad "8" smd roundrect (at 12.52 0.62) (size 0.8 1.24) (layers "F.Cu" "F.Paste" "F.Mask") (roundrect_rratio 0.25) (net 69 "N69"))
  (pad "9" smd roundrect (at 14.46 3.25) (size 1.16 1.25) (layers "F.Cu" "F.Paste" "F.Mask") (roundrect_rratio 0.25) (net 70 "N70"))
  (pad "10" smd roundrect (at 14.46 12.25) (size 1.16 1.25) (layers "F.Cu" "F.Paste" "F.Mask") (roundrect_rratio 0.25) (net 1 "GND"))
  (pad "11" smd roundrect (at 14.86 1.1) (size 1.16 2.2) (layers "F.Cu" "F.Paste" "F.Mask") (roundrect_rratio 0.25) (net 1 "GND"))
  (pad "12" smd roundrect (at 12.66 13.375) (size 1.5 1.15) (layers "F.Cu" "F.Paste" "F.Mask") (roundrect_rratio 0.25) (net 1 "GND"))
  (pad "13" smd roundrect (at 4.88 13.375) (size 1.5 1.15) (layers "F.Cu" "F.Paste" "F.Mask") (roundrect_rratio 0.25) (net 1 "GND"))
  (pad "14" smd roundrect (at 0.575 12.58) (size 1.15 2.2) (layers "F.Cu" "F.Paste" "F.Mask") (roundrect_rratio 0.25) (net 1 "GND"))
  (pad "15" smd roundrect (at 0.575 1.1) (size 1.15 2.2) (layers "F.Cu" "F.Paste" "F.Mask") (roundrect_rratio 0.25) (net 1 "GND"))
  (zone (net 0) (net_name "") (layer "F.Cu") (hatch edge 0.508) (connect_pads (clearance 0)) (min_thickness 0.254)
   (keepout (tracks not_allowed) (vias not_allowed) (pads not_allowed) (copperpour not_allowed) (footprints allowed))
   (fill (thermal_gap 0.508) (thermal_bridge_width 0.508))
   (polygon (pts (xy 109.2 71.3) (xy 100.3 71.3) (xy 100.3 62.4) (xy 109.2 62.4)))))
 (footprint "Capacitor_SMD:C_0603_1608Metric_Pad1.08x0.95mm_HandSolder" (layer "F.Cu") (at 85.3 104.77)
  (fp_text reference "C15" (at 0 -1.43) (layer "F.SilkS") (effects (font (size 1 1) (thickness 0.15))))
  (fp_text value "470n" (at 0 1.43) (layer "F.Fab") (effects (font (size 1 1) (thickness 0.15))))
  (pad "1" smd roundrect locked (at -0.8625 0) (size 1.075 0.95) (layers "F.Cu" "F.Paste" "F.Mask") (roundrect_rratio 0.25)
   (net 10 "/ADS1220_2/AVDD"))
  (pad "2" smd roundrect locked (at 0.8625 0) (size 1.075 0.95) (layers "F.Cu" "F.Paste" "F.Mask") (roundrect_rratio 0.25) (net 1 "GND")))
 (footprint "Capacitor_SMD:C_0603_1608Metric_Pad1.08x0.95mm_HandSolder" (layer "F.Cu") (at 76.2 80.6 -90)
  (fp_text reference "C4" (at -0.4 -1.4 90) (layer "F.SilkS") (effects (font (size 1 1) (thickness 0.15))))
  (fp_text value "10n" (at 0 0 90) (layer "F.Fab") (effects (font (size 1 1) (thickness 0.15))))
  (pad "1" smd roundrect locked (at -0.8625 0 270) (size 1.075 0.95) (layers "F.Cu" "F.Paste" "F.Mask") (roundrect_rratio 0.25)
   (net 23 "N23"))
  (pad "2" smd roundrect locked (at 0.8625 0 270) (size 1.075 0.95) (layers "F.Cu" "F.Paste" "F.Mask") (roundrect_rratio 0.25) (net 1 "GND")))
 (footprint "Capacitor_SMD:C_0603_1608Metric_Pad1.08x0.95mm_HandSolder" (layer "F.Cu") (at 76.2 77.2 -90)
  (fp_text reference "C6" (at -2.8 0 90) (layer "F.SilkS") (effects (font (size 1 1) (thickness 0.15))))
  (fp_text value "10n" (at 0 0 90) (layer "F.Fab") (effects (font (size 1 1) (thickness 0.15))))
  (pad "1" smd roundrect locked (at -0.8625 0 270) (size 1.075 0.95) (layers "F.Cu" "F.Paste" "F.Mask") (roundrect_rratio 0.25)
   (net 1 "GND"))
  (pad "2" smd roundrect locked (at 0.8625 0 270) (size 1.075 0.95) (layers "F.Cu" "F.Paste" "F.Mask") (roundrect_rratio 0.25)
   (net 24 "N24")))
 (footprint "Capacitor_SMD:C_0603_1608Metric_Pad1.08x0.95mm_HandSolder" (layer "F.Cu") (at 90.59 96.97)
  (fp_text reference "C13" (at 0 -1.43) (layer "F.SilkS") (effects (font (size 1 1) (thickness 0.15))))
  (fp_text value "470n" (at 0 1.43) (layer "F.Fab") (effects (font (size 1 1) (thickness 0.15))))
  (pad "1" smd roundrect locked (at -0.8625 0) (size 1.075 0.95) (layers "F.Cu" "F.Paste" "F.Mask") (roundrect_rratio 0.25) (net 2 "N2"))
  (pad "2" smd roundrect locked (at 0.8625 0) (size 1.075 0.95) (layers "F.Cu" "F.Paste" "F.Mask") (roundrect_rratio 0.25) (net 3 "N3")))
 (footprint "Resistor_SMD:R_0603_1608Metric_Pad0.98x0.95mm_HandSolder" (layer "F.Cu") (at 81.2 88.4)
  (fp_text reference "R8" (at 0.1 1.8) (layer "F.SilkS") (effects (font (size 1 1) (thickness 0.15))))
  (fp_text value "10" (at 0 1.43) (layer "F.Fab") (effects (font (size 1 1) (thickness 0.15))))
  (pad "1" smd roundrect locked (at -0.9125 0) (size 0.975 0.95) (layers "F.Cu" "F.Paste" "F.Mask") (roundrect_rratio 0.25)
   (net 5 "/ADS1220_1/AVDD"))
  (pad "2" smd roundrect locked (at 0.9125 0) (size 0.975 0.95) (layers "F.Cu" "F.Paste" "F.Mask") (roundrect_rratio 0.25) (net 11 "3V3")))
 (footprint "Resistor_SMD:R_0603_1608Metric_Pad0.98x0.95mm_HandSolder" (layer "F.Cu") (at 94.94 96.97)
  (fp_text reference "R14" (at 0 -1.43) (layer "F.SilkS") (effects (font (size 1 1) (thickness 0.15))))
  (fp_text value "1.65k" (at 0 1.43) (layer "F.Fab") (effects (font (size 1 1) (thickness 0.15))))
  (pad "1" smd roundrect locked (at -0.9125 0) (size 0.975 0.95) (layers "F.Cu" "F.Paste" "F.Mask") (roundrect_rratio 0.25)
   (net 17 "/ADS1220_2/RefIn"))
  (pad "2" smd roundrect locked (at 0.9125 0) (size 0.975 0.95) (layers "F.Cu" "F.Paste" "F.Mask") (roundrect_rratio 0.25) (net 1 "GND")))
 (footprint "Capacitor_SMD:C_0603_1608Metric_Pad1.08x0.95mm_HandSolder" (layer "F.Cu") (at 76.2 84 90)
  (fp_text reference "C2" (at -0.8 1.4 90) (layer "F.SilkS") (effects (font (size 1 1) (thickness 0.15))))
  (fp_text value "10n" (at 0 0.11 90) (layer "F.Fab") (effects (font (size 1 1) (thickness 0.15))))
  (pad "1" smd roundrect locked (at -0.8625 0 90) (size 1.075 0.95) (layers "F.Cu" "F.Paste" "F.Mask") (roundrect_rratio 0.25)
   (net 25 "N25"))
  (pad "2" smd roundrect locked (at 0.8625 0 90) (size 1.075 0.95) (layers "F.Cu" "F.Paste" "F.Mask") (roundrect_rratio 0.25) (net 1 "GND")))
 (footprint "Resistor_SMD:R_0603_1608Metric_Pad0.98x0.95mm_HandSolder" (layer "F.Cu") (at 89.65 107.01)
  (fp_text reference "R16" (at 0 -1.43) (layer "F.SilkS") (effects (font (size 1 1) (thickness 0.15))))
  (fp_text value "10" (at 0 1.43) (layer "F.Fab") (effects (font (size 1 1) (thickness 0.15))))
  (pad "1" smd roundrect locked (at -0.9125 0) (size 0.975 0.95) (layers "F.Cu" "F.Paste" "F.Mask") (roundrect_rratio 0.25)
   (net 10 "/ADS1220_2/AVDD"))
  (pad "2" smd roundrect locked (at 0.9125 0) (size 0.975 0.95) (layers "F.Cu" "F.Paste" "F.Mask") (roundrect_rratio 0.25) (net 11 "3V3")))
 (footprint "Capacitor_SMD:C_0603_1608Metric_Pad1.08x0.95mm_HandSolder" (layer "F.Cu") (at 80.95 104.77)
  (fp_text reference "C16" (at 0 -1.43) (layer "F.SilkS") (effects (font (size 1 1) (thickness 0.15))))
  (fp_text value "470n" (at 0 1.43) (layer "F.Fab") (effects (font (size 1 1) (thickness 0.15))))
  (pad "1" smd roundrect locked (at -0.8625 0) (size 1.075 0.95) (layers "F.Cu" "F.Paste" "F.Mask") (roundrect_rratio 0.25) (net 11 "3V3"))
  (pad "2" smd roundrect locked (at 0.8625 0) (size 1.075 0.95) (layers "F.Cu" "F.Paste" "F.Mask") (roundrect_rratio 0.25) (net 1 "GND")))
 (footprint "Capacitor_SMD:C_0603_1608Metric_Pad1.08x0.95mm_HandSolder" (layer "F.Cu") (at 74.6 78.8 -90)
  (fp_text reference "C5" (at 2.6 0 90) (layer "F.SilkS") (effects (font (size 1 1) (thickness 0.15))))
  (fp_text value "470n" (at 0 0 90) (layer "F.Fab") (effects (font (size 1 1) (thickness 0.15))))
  (pad "1" smd roundrect locked (at -0.8625 0 270) (size 1.075 0.95) (layers "F.Cu" "F.Paste" "F.Mask") (roundrect_rratio 0.25)
   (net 24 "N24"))
  (pad "2" smd roundrect locked (at 0.8625 0 270) (size 1.075 0.95) (layers "F.Cu" "F.Paste" "F.Mask") (roundrect_rratio 0.25)
   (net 23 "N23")))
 (gr_arc (start 74.5 101.5) (end 74.5 114) (angle 90) (layer "Edge.Cuts") (width 0.1))
 (gr_rect (start 117.9 50.5) (end 117.9 50.5) (layer "Edge.Cuts") (width 0.1) (fill none))
 (gr_arc (start 74.5 72.5) (end 74.5 60) (angle -90) (layer "Edge.Cuts") (width 0.1))
 (gr_line (start 74.5 60) (end 139.5 60) (layer "Edge.Cuts") (width 0.1))
 (gr_arc (start 139.5 72.5) (end 152 72.5) (angle -90) (layer "Edge.Cuts") (width 0.1))
 (gr_line (start 152 72.5) (end 152 101.5) (layer "Edge.Cuts") (width 0.1))
 (gr_line (start 139.5 114) (end 74.5 114) (layer "Edge.Cuts") (width 0.1))
 (gr_line (start 62 101.5) (end 62 72.5) (layer "Edge.Cuts") (width 0.1))
 (gr_arc (start 139.5 101.5) (end 139.5 114) (angle -90) (layer "Edge.Cuts") (width 0.1))
 (segment (start 71.2875 78) (end 69.9125 78) (width 0.25) (layer "F.Cu") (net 1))
 (segment (start 69.9125 78) (end 69.8 77.8875) (width 0.25) (layer "F.Cu") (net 1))
 (segment (start 78.632233 83.107107) (end 77.6 84.13934) (width 0.25) (layer "F.Cu") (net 4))
 (segment (start 74.6 86.4625) (end 76.185 86.4625) (width 0.25) (layer "F.Cu") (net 4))
 (segment (start 73.175 86.4625) (end 73.1125 86.4) (width 0.25) (layer "F.Cu") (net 4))
 (segment (start 77.6 85.4) (end 76.5525 86.4475) (width 0.25) (layer "F.Cu") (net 4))
 (segment (start 76.5525 86.4475) (end 76.2 86.4475) (width 0.25) (layer "F.Cu") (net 4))
 (segment (start 77.6 84.13934) (end 77.6 85.4) (width 0.25) (layer "F.Cu") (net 4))
 (segment (start 74.6 86.4625) (end 73.175 86.4625) (width 0.25) (layer "F.Cu") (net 4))
 (segment (start 76.185 86.4625) (end 76.2 86.4475) (width 0.25) (layer "F.Cu") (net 4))
 (segment (start 74.6 84.7375) (end 73.175 84.7375) (width 0.25) (layer "F.Cu") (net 25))
 (segment (start 74.6 84.7375) (end 76.075 84.7375) (width 0.25) (layer "F.Cu") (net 25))
 (segment (start 76.2 84.8625) (end 78.2 82.8625) (width 0.25) (layer "F.Cu") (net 25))
 (segment (start 78.2 82.8625) (end 78.2 82.125126) (width 0.25) (layer "F.Cu") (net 25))
 (segment (start 73.175 84.7375) (end 73.1125 84.8) (width 0.25) (layer "F.Cu") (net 25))
 (segment (start 78.2 82.125126) (end 78.632233 81.692893) (width 0.25) (layer "F.Cu") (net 25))
 (segment (start 76.075 84.7375) (end 76.2 84.8625) (width 0.25) (layer "F.Cu") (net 25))
 (segment (start 76.125 79.6625) (end 76.2 79.7375) (width 0.25) (layer "F.Cu") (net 23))
 (segment (start 74.6 79.6625) (end 76.125 79.6625) (width 0.25) (layer "F.Cu") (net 23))
 (segment (start 73.175 79.6625) (end 73.1125 79.6) (width 0.25) (layer "F.Cu") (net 23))
 (segment (start 77.383946 79.7375) (end 78.985786 81.33934) (width 0.25) (layer "F.Cu") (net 23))
 (segment (start 76.2 79.7375) (end 77.383946 79.7375) (width 0.25) (layer "F.Cu") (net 23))
 (segment (start 74.6 79.6625) (end 73.175 79.6625) (width 0.25) (layer "F.Cu") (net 23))
 (segment (start 74.6 77.9375) (end 73.175 77.9375) (width 0.25) (layer "F.Cu") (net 24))
 (segment (start 73.175 77.9375) (end 73.1125 78) (width 0.25) (layer "F.Cu") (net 24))
 (segment (start 76.416054 78.0625) (end 76.2 78.0625) (width 0.25) (layer "F.Cu") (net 24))
 (segment (start 79.33934 80.985786) (end 76.416054 78.0625) (width 0.25) (layer "F.Cu") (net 24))
 (segment (start 74.6 77.9375) (end 76.075 77.9375) (width 0.25) (layer "F.Cu") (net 24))
 (segment (start 76.075 77.9375) (end 76.2 78.0625) (width 0.25) (layer "F.Cu") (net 24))
 (segment (start 71.2875 88) (end 71.2875 86.4) (width 0.25) (layer "F.Cu") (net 21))
 (segment (start 71.2875 84.8) (end 71.2875 83.2) (width 0.25) (layer "F.Cu") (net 19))
 (segment (start 71.2875 79.6) (end 69.9125 79.6) (width 0.25) (layer "F.Cu") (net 22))
 (segment (start 69.9125 79.6) (end 69.8 79.7125) (width 0.25) (layer "F.Cu") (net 22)))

